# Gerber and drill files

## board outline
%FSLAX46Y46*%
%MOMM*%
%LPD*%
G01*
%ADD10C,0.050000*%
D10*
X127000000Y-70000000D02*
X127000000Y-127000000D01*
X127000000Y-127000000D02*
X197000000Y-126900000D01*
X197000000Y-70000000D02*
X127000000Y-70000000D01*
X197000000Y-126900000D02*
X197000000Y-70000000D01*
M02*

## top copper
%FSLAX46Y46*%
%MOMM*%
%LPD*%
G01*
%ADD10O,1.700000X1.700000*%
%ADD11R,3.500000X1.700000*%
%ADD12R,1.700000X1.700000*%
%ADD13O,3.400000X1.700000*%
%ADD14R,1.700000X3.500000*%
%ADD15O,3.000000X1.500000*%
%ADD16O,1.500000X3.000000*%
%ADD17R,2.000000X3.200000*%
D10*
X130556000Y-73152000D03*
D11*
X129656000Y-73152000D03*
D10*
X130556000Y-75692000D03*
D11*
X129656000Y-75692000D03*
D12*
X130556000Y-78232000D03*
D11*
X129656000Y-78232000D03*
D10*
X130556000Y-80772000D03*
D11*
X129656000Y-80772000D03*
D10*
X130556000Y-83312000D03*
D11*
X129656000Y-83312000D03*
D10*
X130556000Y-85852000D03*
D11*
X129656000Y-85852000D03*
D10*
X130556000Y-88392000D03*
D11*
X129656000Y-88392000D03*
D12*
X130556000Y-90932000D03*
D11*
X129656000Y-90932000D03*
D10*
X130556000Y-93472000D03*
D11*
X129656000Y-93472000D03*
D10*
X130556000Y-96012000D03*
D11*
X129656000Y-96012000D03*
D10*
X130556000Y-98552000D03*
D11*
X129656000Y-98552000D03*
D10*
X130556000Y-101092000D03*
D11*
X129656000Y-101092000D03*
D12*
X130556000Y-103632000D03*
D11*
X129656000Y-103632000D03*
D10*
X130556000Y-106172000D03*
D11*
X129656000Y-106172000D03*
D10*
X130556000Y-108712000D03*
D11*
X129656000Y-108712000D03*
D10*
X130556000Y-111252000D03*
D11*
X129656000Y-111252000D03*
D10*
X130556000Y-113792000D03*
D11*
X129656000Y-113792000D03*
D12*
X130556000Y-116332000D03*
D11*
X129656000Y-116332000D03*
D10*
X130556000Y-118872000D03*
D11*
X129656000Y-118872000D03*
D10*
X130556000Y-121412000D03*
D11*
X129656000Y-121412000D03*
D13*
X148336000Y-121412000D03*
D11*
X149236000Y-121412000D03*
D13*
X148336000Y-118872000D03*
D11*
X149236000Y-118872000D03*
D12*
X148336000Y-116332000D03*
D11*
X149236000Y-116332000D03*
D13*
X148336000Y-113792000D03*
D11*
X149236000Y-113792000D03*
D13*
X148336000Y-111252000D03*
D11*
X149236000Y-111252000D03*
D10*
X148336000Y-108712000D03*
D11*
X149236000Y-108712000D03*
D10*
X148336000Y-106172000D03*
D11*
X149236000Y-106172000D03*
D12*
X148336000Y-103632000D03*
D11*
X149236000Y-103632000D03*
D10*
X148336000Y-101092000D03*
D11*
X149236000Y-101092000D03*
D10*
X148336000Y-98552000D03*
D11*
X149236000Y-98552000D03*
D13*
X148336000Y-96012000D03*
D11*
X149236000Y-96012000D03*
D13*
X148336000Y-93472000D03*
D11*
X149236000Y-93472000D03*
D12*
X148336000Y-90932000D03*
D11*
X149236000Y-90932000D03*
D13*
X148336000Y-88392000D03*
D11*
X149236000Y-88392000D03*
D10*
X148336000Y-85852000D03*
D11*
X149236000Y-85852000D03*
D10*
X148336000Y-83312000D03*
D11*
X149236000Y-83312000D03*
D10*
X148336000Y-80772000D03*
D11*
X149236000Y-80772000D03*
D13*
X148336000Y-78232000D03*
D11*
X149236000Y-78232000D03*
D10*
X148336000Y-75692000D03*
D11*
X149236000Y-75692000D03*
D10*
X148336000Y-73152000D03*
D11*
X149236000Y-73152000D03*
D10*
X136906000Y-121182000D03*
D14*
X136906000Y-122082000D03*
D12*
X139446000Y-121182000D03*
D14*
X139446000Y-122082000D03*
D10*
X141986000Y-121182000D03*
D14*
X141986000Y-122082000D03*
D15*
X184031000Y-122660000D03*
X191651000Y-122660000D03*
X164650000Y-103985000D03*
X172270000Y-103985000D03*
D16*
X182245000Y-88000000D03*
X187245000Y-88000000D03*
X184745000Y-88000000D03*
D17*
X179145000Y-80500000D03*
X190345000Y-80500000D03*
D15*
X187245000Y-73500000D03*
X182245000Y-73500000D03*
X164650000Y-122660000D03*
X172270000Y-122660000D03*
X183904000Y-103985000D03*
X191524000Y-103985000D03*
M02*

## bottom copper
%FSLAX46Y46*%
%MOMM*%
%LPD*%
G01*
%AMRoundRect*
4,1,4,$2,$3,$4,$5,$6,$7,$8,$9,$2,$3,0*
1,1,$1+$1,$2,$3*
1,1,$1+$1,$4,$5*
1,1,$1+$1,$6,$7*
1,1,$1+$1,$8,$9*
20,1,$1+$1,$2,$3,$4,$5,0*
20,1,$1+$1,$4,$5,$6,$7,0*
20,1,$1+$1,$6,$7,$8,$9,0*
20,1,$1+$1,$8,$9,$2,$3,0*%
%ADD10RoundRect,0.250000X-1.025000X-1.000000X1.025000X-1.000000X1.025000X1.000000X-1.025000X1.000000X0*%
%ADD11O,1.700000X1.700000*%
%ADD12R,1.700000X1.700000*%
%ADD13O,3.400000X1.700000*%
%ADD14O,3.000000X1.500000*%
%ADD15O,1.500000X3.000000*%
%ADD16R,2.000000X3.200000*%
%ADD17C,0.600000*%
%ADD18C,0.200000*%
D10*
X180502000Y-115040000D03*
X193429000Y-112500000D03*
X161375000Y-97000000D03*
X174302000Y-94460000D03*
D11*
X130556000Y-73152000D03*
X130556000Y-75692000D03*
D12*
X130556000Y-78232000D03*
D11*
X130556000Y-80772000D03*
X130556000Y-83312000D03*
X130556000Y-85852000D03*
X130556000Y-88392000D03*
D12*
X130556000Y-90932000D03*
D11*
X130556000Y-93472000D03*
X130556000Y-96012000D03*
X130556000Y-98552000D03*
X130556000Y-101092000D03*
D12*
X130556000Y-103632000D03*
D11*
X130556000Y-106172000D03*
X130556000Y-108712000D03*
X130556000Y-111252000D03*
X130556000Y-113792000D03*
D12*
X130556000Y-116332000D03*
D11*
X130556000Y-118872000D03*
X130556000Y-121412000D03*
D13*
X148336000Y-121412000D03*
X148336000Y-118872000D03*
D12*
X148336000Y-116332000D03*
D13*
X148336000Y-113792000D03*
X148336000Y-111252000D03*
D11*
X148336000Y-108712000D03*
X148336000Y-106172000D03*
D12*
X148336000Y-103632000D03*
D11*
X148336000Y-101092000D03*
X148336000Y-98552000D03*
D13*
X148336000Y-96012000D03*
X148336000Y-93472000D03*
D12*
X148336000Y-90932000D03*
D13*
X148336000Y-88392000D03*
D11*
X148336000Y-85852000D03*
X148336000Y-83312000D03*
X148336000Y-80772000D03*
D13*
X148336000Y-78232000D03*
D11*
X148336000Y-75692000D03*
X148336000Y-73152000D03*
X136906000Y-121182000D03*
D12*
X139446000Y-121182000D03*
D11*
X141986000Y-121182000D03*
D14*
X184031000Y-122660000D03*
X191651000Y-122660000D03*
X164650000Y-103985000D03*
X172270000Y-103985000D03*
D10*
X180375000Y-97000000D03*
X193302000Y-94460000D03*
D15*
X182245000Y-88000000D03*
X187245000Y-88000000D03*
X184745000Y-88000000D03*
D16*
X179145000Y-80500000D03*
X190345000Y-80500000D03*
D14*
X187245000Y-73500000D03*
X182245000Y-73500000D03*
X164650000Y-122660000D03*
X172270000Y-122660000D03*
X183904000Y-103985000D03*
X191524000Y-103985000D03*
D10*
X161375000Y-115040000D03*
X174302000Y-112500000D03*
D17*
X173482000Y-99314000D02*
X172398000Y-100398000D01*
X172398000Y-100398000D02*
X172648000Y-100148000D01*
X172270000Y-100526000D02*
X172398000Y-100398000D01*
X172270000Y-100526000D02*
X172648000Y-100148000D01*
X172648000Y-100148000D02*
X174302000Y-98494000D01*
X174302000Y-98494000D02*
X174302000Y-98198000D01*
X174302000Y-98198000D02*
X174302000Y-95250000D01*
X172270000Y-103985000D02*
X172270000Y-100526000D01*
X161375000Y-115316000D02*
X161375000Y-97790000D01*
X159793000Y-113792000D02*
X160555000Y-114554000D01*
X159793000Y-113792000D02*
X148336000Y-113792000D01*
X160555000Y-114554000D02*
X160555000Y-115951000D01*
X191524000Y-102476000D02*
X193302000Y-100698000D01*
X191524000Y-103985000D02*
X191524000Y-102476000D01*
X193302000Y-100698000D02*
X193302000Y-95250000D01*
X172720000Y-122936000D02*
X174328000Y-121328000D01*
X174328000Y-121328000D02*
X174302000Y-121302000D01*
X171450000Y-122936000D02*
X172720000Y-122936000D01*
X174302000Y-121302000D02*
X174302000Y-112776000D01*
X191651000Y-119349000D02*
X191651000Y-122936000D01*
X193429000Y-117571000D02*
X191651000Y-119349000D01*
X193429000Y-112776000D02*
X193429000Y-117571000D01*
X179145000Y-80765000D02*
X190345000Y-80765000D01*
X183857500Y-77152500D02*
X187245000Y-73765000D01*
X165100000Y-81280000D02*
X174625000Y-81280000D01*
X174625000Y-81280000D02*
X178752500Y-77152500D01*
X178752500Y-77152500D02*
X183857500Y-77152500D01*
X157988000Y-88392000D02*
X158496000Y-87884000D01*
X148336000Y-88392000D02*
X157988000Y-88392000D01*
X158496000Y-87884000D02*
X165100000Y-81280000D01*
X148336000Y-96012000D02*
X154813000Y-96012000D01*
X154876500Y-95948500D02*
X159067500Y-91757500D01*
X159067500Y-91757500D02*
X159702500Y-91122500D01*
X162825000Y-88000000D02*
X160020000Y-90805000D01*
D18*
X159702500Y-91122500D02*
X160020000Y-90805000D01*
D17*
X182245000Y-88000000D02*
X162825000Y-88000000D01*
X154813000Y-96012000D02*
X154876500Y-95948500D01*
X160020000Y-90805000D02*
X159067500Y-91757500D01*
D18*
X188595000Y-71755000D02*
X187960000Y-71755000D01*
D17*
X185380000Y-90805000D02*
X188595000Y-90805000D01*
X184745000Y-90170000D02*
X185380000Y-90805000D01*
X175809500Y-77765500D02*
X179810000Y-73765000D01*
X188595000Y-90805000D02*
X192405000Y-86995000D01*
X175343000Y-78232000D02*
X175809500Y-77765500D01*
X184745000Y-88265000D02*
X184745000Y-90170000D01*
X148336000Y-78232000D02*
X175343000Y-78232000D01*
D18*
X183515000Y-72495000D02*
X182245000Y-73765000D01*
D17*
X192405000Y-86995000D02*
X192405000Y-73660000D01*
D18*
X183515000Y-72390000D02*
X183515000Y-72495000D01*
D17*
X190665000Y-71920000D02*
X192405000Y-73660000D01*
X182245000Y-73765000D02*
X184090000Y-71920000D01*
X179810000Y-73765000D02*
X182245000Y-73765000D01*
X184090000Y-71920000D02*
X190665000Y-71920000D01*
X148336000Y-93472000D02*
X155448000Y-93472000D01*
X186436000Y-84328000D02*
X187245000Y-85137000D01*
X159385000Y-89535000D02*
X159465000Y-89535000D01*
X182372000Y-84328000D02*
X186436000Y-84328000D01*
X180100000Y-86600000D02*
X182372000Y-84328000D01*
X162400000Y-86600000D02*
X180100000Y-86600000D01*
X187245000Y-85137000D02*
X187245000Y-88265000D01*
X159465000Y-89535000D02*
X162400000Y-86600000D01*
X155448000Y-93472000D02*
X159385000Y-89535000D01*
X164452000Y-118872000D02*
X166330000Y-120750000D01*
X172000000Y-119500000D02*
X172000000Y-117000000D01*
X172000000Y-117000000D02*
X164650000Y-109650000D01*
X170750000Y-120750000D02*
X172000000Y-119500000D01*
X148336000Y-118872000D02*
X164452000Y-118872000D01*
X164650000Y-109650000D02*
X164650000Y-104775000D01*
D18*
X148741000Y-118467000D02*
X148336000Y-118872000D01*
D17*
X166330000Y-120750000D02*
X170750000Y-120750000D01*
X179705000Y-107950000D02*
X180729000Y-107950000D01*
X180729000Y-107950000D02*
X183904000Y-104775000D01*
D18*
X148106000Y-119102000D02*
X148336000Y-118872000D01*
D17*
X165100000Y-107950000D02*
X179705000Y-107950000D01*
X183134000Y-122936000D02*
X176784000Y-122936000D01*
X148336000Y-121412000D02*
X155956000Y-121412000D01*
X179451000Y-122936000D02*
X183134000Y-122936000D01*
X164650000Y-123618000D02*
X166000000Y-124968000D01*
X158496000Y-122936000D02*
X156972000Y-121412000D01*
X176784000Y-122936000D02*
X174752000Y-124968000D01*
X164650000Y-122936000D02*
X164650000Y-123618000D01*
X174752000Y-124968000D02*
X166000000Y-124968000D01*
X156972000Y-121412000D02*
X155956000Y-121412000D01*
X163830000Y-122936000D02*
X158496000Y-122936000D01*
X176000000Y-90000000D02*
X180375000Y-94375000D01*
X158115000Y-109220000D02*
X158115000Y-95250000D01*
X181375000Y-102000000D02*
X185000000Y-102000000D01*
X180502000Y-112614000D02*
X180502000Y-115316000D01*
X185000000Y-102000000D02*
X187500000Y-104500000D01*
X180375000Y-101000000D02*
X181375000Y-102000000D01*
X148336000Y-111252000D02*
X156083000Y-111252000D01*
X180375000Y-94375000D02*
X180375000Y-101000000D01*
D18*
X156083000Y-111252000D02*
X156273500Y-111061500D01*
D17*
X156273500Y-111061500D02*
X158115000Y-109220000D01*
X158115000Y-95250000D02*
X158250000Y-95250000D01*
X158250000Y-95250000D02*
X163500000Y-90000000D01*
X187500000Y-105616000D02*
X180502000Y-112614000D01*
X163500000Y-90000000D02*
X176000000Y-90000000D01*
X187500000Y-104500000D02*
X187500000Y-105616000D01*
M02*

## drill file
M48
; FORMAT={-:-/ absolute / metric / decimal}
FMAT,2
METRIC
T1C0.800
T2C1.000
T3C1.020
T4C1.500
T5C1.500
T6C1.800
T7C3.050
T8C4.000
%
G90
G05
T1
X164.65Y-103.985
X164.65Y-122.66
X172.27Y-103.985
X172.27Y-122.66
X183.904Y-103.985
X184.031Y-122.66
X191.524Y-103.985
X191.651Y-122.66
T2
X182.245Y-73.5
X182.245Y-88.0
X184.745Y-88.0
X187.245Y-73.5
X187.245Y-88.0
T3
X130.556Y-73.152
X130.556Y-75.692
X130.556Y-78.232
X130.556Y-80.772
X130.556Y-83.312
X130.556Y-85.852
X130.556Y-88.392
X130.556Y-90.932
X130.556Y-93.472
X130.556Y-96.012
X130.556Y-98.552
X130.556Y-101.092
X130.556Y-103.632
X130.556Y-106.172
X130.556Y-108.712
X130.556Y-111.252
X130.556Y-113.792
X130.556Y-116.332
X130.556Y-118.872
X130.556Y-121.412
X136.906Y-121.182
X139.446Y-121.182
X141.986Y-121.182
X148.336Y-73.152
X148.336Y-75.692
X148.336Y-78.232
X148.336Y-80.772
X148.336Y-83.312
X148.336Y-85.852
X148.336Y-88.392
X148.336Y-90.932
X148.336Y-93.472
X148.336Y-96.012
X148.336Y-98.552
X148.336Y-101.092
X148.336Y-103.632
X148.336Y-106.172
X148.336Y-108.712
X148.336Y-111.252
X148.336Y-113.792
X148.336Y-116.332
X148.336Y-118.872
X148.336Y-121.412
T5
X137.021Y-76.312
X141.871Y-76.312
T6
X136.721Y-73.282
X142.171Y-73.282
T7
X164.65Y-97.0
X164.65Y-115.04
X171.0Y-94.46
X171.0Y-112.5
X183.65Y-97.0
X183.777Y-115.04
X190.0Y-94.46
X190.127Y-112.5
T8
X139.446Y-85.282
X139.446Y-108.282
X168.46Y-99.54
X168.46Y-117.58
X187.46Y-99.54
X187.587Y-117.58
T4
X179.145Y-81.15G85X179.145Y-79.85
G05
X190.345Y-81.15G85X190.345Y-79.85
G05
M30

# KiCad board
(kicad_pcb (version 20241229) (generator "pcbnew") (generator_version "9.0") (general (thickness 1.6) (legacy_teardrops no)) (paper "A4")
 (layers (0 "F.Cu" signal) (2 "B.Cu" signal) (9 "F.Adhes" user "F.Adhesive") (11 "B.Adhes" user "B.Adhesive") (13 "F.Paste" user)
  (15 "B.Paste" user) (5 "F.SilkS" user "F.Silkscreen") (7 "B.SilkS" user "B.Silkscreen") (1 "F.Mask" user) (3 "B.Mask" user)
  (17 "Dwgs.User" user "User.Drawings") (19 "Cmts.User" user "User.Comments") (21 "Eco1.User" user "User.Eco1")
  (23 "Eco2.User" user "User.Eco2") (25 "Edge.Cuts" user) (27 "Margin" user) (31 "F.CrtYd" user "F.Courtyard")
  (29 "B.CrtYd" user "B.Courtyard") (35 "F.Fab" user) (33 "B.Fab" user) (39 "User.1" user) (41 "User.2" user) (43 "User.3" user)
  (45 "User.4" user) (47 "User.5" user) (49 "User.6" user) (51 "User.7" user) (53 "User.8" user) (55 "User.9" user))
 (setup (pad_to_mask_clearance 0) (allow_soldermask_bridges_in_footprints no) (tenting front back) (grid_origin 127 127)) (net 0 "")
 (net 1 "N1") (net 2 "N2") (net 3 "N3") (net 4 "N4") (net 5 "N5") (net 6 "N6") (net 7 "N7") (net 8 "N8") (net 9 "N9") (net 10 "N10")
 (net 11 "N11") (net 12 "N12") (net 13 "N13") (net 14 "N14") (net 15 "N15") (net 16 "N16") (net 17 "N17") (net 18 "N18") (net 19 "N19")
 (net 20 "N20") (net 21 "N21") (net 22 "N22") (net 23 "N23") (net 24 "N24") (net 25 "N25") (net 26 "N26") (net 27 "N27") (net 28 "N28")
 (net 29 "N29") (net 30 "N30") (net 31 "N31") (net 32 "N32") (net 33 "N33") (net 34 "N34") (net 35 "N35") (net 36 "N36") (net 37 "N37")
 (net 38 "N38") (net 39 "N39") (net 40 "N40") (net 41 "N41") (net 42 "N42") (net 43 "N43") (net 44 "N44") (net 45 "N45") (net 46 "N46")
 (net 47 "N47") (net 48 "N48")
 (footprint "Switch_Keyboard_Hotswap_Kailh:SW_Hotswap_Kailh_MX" (layer "F.Cu") (at 187.587 117.58)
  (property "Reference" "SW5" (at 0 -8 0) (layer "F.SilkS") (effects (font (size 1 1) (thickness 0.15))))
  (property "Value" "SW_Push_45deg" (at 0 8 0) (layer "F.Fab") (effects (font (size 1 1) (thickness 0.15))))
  (pad "" np_thru_hole circle (at -3.81 -2.54) (size 3.05 3.05) (drill 3.05) (layers "*.Cu" "*.Mask"))
  (pad "" np_thru_hole circle (at 0 0) (size 4 4) (drill 4) (layers "*.Cu" "*.Mask"))
  (pad "" np_thru_hole circle (at 2.54 -5.08) (size 3.05 3.05) (drill 3.05) (layers "*.Cu" "*.Mask"))
  (pad "1" smd roundrect (at -7.085 -2.54) (size 2.55 2.5) (layers "B.Cu" "B.Mask" "B.Paste") (roundrect_rratio 0.1) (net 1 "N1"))
  (pad "2" smd roundrect (at 5.842 -5.08) (size 2.55 2.5) (layers "B.Cu" "B.Mask" "B.Paste") (roundrect_rratio 0.1) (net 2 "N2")))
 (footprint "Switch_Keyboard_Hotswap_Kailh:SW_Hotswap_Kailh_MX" (layer "F.Cu") (at 168.46 99.54)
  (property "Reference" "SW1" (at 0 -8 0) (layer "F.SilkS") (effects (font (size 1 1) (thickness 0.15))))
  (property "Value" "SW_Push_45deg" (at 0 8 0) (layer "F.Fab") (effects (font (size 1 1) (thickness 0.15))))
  (pad "" np_thru_hole circle (at -3.81 -2.54) (size 3.05 3.05) (drill 3.05) (layers "*.Cu" "*.Mask"))
  (pad "" np_thru_hole circle (at 0 0) (size 4 4) (drill 4) (layers "*.Cu" "*.Mask"))
  (pad "" np_thru_hole circle (at 2.54 -5.08) (size 3.05 3.05) (drill 3.05) (layers "*.Cu" "*.Mask"))
  (pad "1" smd roundrect (at -7.085 -2.54) (size 2.55 2.5) (layers "B.Cu" "B.Mask" "B.Paste") (roundrect_rratio 0.1) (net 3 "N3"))
  (pad "2" smd roundrect (at 5.842 -5.08) (size 2.55 2.5) (layers "B.Cu" "B.Mask" "B.Paste") (roundrect_rratio 0.1) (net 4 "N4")))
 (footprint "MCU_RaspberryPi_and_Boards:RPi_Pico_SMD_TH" (layer "F.Cu") (at 139.446 97.282)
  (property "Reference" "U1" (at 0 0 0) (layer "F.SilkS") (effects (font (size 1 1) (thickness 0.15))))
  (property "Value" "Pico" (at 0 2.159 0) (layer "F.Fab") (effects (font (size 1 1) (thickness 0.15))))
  (pad "" np_thru_hole oval (at -2.725 -24) (size 1.8 1.8) (drill 1.8) (layers "*.Cu" "*.Mask"))
  (pad "" np_thru_hole oval (at -2.425 -20.97) (size 1.5 1.5) (drill 1.5) (layers "*.Cu" "*.Mask"))
  (pad "" np_thru_hole oval (at 0 -12) (size 4 4) (drill 4) (layers "*.Cu" "*.Mask"))
  (pad "" np_thru_hole oval (at 0 11) (size 4 4) (drill 4) (layers "*.Cu" "*.Mask"))
  (pad "" np_thru_hole oval (at 2.425 -20.97) (size 1.5 1.5) (drill 1.5) (layers "*.Cu" "*.Mask"))
  (pad "" np_thru_hole oval (at 2.725 -24) (size 1.8 1.8) (drill 1.8) (layers "*.Cu" "*.Mask"))
  (pad "1" thru_hole oval (at -8.89 -24.13) (size 1.7 1.7) (drill 1.02) (layers "*.Cu" "*.Mask") (remove_unused_layers no) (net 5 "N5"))
  (pad "1" smd rect (at -8.89 -24.13) (size 3.5 1.7) (drill (offset -0.9 0)) (layers "F.Cu" "F.Mask") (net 5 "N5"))
  (pad "2" thru_hole oval (at -8.89 -21.59) (size 1.7 1.7) (drill 1.02) (layers "*.Cu" "*.Mask") (remove_unused_layers no) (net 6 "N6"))
  (pad "2" smd rect (at -8.89 -21.59) (size 3.5 1.7) (drill (offset -0.9 0)) (layers "F.Cu" "F.Mask") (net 6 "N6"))
  (pad "3" thru_hole rect (at -8.89 -19.05) (size 1.7 1.7) (drill 1.02) (layers "*.Cu" "*.Mask") (remove_unused_layers no) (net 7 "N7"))
  (pad "3" smd rect (at -8.89 -19.05) (size 3.5 1.7) (drill (offset -0.9 0)) (layers "F.Cu" "F.Mask") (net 7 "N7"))
  (pad "4" thru_hole oval (at -8.89 -16.51) (size 1.7 1.7) (drill 1.02) (layers "*.Cu" "*.Mask") (remove_unused_layers no) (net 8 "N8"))
  (pad "4" smd rect (at -8.89 -16.51) (size 3.5 1.7) (drill (offset -0.9 0)) (layers "F.Cu" "F.Mask") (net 8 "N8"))
  (pad "5" thru_hole oval (at -8.89 -13.97) (size 1.7 1.7) (drill 1.02) (layers "*.Cu" "*.Mask") (remove_unused_layers no) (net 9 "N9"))
  (pad "5" smd rect (at -8.89 -13.97) (size 3.5 1.7) (drill (offset -0.9 0)) (layers "F.Cu" "F.Mask") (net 9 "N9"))
  (pad "6" thru_hole oval (at -8.89 -11.43) (size 1.7 1.7) (drill 1.02) (layers "*.Cu" "*.Mask") (remove_unused_layers no) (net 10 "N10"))
  (pad "6" smd rect (at -8.89 -11.43) (size 3.5 1.7) (drill (offset -0.9 0)) (layers "F.Cu" "F.Mask") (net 10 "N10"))
  (pad "7" thru_hole oval (at -8.89 -8.89) (size 1.7 1.7) (drill 1.02) (layers "*.Cu" "*.Mask") (remove_unused_layers no) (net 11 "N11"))
  (pad "7" smd rect (at -8.89 -8.89) (size 3.5 1.7) (drill (offset -0.9 0)) (layers "F.Cu" "F.Mask") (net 11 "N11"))
  (pad "8" thru_hole rect (at -8.89 -6.35) (size 1.7 1.7) (drill 1.02) (layers "*.Cu" "*.Mask") (remove_unused_layers no) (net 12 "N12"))
  (pad "8" smd rect (at -8.89 -6.35) (size 3.5 1.7) (drill (offset -0.9 0)) (layers "F.Cu" "F.Mask") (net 12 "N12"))
  (pad "9" thru_hole oval (at -8.89 -3.81) (size 1.7 1.7) (drill 1.02) (layers "*.Cu" "*.Mask") (remove_unused_layers no) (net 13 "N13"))
  (pad "9" smd rect (at -8.89 -3.81) (size 3.5 1.7) (drill (offset -0.9 0)) (layers "F.Cu" "F.Mask") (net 13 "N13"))
  (pad "10" thru_hole oval (at -8.89 -1.27) (size 1.7 1.7) (drill 1.02) (layers "*.Cu" "*.Mask") (remove_unused_layers no) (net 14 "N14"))
  (pad "10" smd rect (at -8.89 -1.27) (size 3.5 1.7) (drill (offset -0.9 0)) (layers "F.Cu" "F.Mask") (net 14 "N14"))
  (pad "11" thru_hole oval (at -8.89 1.27) (size 1.7 1.7) (drill 1.02) (layers "*.Cu" "*.Mask") (remove_unused_layers no) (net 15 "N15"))
  (pad "11" smd rect (at -8.89 1.27) (size 3.5 1.7) (drill (offset -0.9 0)) (layers "F.Cu" "F.Mask") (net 15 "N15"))
  (pad "12" thru_hole oval (at -8.89 3.81) (size 1.7 1.7) (drill 1.02) (layers "*.Cu" "*.Mask") (remove_unused_layers no) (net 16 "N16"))
  (pad "12" smd rect (at -8.89 3.81) (size 3.5 1.7) (drill (offset -0.9 0)) (layers "F.Cu" "F.Mask") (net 16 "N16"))
  (pad "13" thru_hole rect (at -8.89 6.35) (size 1.7 1.7) (drill 1.02) (layers "*.Cu" "*.Mask") (remove_unused_layers no) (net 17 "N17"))
  (pad "13" smd rect (at -8.89 6.35) (size 3.5 1.7) (drill (offset -0.9 0)) (layers "F.Cu" "F.Mask") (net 17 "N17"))
  (pad "14" thru_hole oval (at -8.89 8.89) (size 1.7 1.7) (drill 1.02) (layers "*.Cu" "*.Mask") (remove_unused_layers no) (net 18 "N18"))
  (pad "14" smd rect (at -8.89 8.89) (size 3.5 1.7) (drill (offset -0.9 0)) (layers "F.Cu" "F.Mask") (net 18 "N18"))
  (pad "15" thru_hole oval (at -8.89 11.43) (size 1.7 1.7) (drill 1.02) (layers "*.Cu" "*.Mask") (remove_unused_layers no) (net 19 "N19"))
  (pad "15" smd rect (at -8.89 11.43) (size 3.5 1.7) (drill (offset -0.9 0)) (layers "F.Cu" "F.Mask") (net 19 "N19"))
  (pad "16" thru_hole oval (at -8.89 13.97) (size 1.7 1.7) (drill 1.02) (layers "*.Cu" "*.Mask") (remove_unused_layers no) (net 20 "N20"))
  (pad "16" smd rect (at -8.89 13.97) (size 3.5 1.7) (drill (offset -0.9 0)) (layers "F.Cu" "F.Mask") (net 20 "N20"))
  (pad "17" thru_hole oval (at -8.89 16.51) (size 1.7 1.7) (drill 1.02) (layers "*.Cu" "*.Mask") (remove_unused_layers no) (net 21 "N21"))
  (pad "17" smd rect (at -8.89 16.51) (size 3.5 1.7) (drill (offset -0.9 0)) (layers "F.Cu" "F.Mask") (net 21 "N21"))
  (pad "18" thru_hole rect (at -8.89 19.05) (size 1.7 1.7) (drill 1.02) (layers "*.Cu" "*.Mask") (remove_unused_layers no) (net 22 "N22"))
  (pad "18" smd rect (at -8.89 19.05) (size 3.5 1.7) (drill (offset -0.9 0)) (layers "F.Cu" "F.Mask") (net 22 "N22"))
  (pad "19" thru_hole oval (at -8.89 21.59) (size 1.7 1.7) (drill 1.02) (layers "*.Cu" "*.Mask") (remove_unused_layers no) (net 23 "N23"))
  (pad "19" smd rect (at -8.89 21.59) (size 3.5 1.7) (drill (offset -0.9 0)) (layers "F.Cu" "F.Mask") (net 23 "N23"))
  (pad "20" thru_hole oval (at -8.89 24.13) (size 1.7 1.7) (drill 1.02) (layers "*.Cu" "*.Mask") (remove_unused_layers no) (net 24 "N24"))
  (pad "20" smd rect (at -8.89 24.13) (size 3.5 1.7) (drill (offset -0.9 0)) (layers "F.Cu" "F.Mask") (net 24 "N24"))
  (pad "21" thru_hole oval (at 8.89 24.13) (size 3.4 1.7) (drill 1.02) (layers "*.Cu" "*.Mask") (remove_unused_layers no) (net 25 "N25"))
  (pad "21" smd rect (at 8.89 24.13) (size 3.5 1.7) (drill (offset 0.9 0)) (layers "F.Cu" "F.Mask") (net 25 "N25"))
  (pad "22" thru_hole oval (at 8.89 21.59) (size 3.4 1.7) (drill 1.02) (layers "*.Cu" "*.Mask") (remove_unused_layers no) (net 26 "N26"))
  (pad "22" smd rect (at 8.89 21.59) (size 3.5 1.7) (drill (offset 0.9 0)) (layers "F.Cu" "F.Mask") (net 26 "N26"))
  (pad "23" thru_hole rect (at 8.89 19.05) (size 1.7 1.7) (drill 1.02) (layers "*.Cu" "*.Mask") (remove_unused_layers no) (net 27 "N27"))
  (pad "23" smd rect (at 8.89 19.05) (size 3.5 1.7) (drill (offset 0.9 0)) (layers "F.Cu" "F.Mask") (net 27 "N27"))
  (pad "24" thru_hole oval (at 8.89 16.51) (size 3.4 1.7) (drill 1.02) (layers "*.Cu" "*.Mask") (remove_unused_layers no) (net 3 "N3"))
  (pad "24" smd rect (at 8.89 16.51) (size 3.5 1.7) (drill (offset 0.9 0)) (layers "F.Cu" "F.Mask") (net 3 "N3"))
  (pad "25" thru_hole oval (at 8.89 13.97) (size 3.4 1.7) (drill 1.02) (layers "*.Cu" "*.Mask") (remove_unused_layers no) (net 1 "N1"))
  (pad "25" smd rect (at 8.89 13.97) (size 3.5 1.7) (drill (offset 0.9 0)) (layers "F.Cu" "F.Mask") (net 1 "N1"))
  (pad "26" thru_hole oval (at 8.89 11.43) (size 1.7 1.7) (drill 1.02) (layers "*.Cu" "*.Mask") (remove_unused_layers no) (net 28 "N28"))
  (pad "26" smd rect (at 8.89 11.43) (size 3.5 1.7) (drill (offset 0.9 0)) (layers "F.Cu" "F.Mask") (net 28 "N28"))
  (pad "27" thru_hole oval (at 8.89 8.89) (size 1.7 1.7) (drill 1.02) (layers "*.Cu" "*.Mask") (remove_unused_layers no) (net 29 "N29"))
  (pad "27" smd rect (at 8.89 8.89) (size 3.5 1.7) (drill (offset 0.9 0)) (layers "F.Cu" "F.Mask") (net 29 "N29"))
  (pad "28" thru_hole rect (at 8.89 6.35) (size 1.7 1.7) (drill 1.02) (layers "*.Cu" "*.Mask") (remove_unused_layers no) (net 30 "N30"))
  (pad "28" smd rect (at 8.89 6.35) (size 3.5 1.7) (drill (offset 0.9 0)) (layers "F.Cu" "F.Mask") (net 30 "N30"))
  (pad "29" thru_hole oval (at 8.89 3.81) (size 1.7 1.7) (drill 1.02) (layers "*.Cu" "*.Mask") (remove_unused_layers no) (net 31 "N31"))
  (pad "29" smd rect (at 8.89 3.81) (size 3.5 1.7) (drill (offset 0.9 0)) (layers "F.Cu" "F.Mask") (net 31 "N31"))
  (pad "30" thru_hole oval (at 8.89 1.27) (size 1.7 1.7) (drill 1.02) (layers "*.Cu" "*.Mask") (remove_unused_layers no) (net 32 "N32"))
  (pad "30" smd rect (at 8.89 1.27) (size 3.5 1.7) (drill (offset 0.9 0)) (layers "F.Cu" "F.Mask") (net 32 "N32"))
  (pad "31" thru_hole oval (at 8.89 -1.27) (size 3.4 1.7) (drill 1.02) (layers "*.Cu" "*.Mask") (remove_unused_layers no) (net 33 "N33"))
  (pad "31" smd rect (at 8.89 -1.27) (size 3.5 1.7) (drill (offset 0.9 0)) (layers "F.Cu" "F.Mask") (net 33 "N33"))
  (pad "32" thru_hole oval (at 8.89 -3.81) (size 3.4 1.7) (drill 1.02) (layers "*.Cu" "*.Mask") (remove_unused_layers no) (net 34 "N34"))
  (pad "32" smd rect (at 8.89 -3.81) (size 3.5 1.7) (drill (offset 0.9 0)) (layers "F.Cu" "F.Mask") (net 34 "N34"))
  (pad "33" thru_hole rect (at 8.89 -6.35) (size 1.7 1.7) (drill 1.02) (layers "*.Cu" "*.Mask") (remove_unused_layers no) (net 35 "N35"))
  (pad "33" smd rect (at 8.89 -6.35) (size 3.5 1.7) (drill (offset 0.9 0)) (layers "F.Cu" "F.Mask") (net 35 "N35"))
  (pad "34" thru_hole oval (at 8.89 -8.89) (size 3.4 1.7) (drill 1.02) (layers "*.Cu" "*.Mask") (remove_unused_layers no) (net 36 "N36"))
  (pad "34" smd rect (at 8.89 -8.89) (size 3.5 1.7) (drill (offset 0.9 0)) (layers "F.Cu" "F.Mask") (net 36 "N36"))
  (pad "35" thru_hole oval (at 8.89 -11.43) (size 1.7 1.7) (drill 1.02) (layers "*.Cu" "*.Mask") (remove_unused_layers no) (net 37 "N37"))
  (pad "35" smd rect (at 8.89 -11.43) (size 3.5 1.7) (drill (offset 0.9 0)) (layers "F.Cu" "F.Mask") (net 37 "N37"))
  (pad "36" thru_hole oval (at 8.89 -13.97) (size 1.7 1.7) (drill 1.02) (layers "*.Cu" "*.Mask") (remove_unused_layers no) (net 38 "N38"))
  (pad "36" smd rect (at 8.89 -13.97) (size 3.5 1.7) (drill (offset 0.9 0)) (layers "F.Cu" "F.Mask") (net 38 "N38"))
  (pad "37" thru_hole oval (at 8.89 -16.51) (size 1.7 1.7) (drill 1.02) (layers "*.Cu" "*.Mask") (remove_unused_layers no) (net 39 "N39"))
  (pad "37" smd rect (at 8.89 -16.51) (size 3.5 1.7) (drill (offset 0.9 0)) (layers "F.Cu" "F.Mask") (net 39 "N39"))
  (pad "38" thru_hole oval (at 8.89 -19.05) (size 3.4 1.7) (drill 1.02) (layers "*.Cu" "*.Mask") (remove_unused_layers no) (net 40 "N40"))
  (pad "38" smd rect (at 8.89 -19.05) (size 3.5 1.7) (drill (offset 0.9 0)) (layers "F.Cu" "F.Mask") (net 40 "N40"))
  (pad "39" thru_hole oval (at 8.89 -21.59) (size 1.7 1.7) (drill 1.02) (layers "*.Cu" "*.Mask") (remove_unused_layers no) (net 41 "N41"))
  (pad "39" smd rect (at 8.89 -21.59) (size 3.5 1.7) (drill (offset 0.9 0)) (layers "F.Cu" "F.Mask") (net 41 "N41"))
  (pad "40" thru_hole oval (at 8.89 -24.13) (size 1.7 1.7) (drill 1.02) (layers "*.Cu" "*.Mask") (remove_unused_layers no) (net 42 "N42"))
  (pad "40" smd rect (at 8.89 -24.13) (size 3.5 1.7) (drill (offset 0.9 0)) (layers "F.Cu" "F.Mask") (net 42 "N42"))
  (pad "41" thru_hole oval (at -2.54 23.9) (size 1.7 1.7) (drill 1.02) (layers "*.Cu" "*.Mask") (remove_unused_layers no) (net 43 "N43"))
  (pad "41" smd rect (at -2.54 23.9 90) (size 3.5 1.7) (drill (offset -0.9 0)) (layers "F.Cu" "F.Mask") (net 43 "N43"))
  (pad "42" thru_hole rect (at 0 23.9) (size 1.7 1.7) (drill 1.02) (layers "*.Cu" "*.Mask") (remove_unused_layers no) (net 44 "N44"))
  (pad "42" smd rect (at 0 23.9 90) (size 3.5 1.7) (drill (offset -0.9 0)) (layers "F.Cu" "F.Mask") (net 44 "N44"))
  (pad "43" thru_hole oval (at 2.54 23.9) (size 1.7 1.7) (drill 1.02) (layers "*.Cu" "*.Mask") (remove_unused_layers no) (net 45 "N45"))
  (pad "43" smd rect (at 2.54 23.9 90) (size 3.5 1.7) (drill (offset -0.9 0)) (layers "F.Cu" "F.Mask") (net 45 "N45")))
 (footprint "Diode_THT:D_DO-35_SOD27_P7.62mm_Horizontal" (layer "F.Cu") (at 184.031 122.66)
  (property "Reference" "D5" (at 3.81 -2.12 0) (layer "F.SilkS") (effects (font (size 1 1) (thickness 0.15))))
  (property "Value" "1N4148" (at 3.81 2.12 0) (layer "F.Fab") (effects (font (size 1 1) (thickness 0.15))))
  (pad "1" thru_hole oval (at 0 0) (size 3 1.5) (drill 0.8) (layers "*.Cu" "*.Mask") (remove_unused_layers no) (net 25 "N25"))
  (pad "2" thru_hole oval (at 7.62 0) (size 3 1.5) (drill 0.8) (layers "*.Cu" "*.Mask") (remove_unused_layers no) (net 2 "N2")))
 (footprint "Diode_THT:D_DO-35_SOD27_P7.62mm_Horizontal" (layer "F.Cu") (at 164.65 103.985)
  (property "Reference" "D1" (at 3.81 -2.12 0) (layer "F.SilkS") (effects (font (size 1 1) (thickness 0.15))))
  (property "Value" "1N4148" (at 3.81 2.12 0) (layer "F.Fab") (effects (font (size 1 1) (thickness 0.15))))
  (pad "1" thru_hole oval (at 0 0) (size 3 1.5) (drill 0.8) (layers "*.Cu" "*.Mask") (remove_unused_layers no) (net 26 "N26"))
  (pad "2" thru_hole oval (at 7.62 0) (size 3 1.5) (drill 0.8) (layers "*.Cu" "*.Mask") (remove_unused_layers no) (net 4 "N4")))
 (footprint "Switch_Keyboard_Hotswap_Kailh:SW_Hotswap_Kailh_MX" (layer "F.Cu") (at 187.46 99.54)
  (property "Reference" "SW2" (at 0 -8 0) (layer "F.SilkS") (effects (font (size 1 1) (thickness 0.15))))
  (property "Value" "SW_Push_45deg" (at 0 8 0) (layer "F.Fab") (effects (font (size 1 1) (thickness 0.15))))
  (pad "" np_thru_hole circle (at -3.81 -2.54) (size 3.05 3.05) (drill 3.05) (layers "*.Cu" "*.Mask"))
  (pad "" np_thru_hole circle (at 0 0) (size 4 4) (drill 4) (layers "*.Cu" "*.Mask"))
  (pad "" np_thru_hole circle (at 2.54 -5.08) (size 3.05 3.05) (drill 3.05) (layers "*.Cu" "*.Mask"))
  (pad "1" smd roundrect (at -7.085 -2.54) (size 2.55 2.5) (layers "B.Cu" "B.Mask" "B.Paste") (roundrect_rratio 0.1) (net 1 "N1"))
  (pad "2" smd roundrect (at 5.842 -5.08) (size 2.55 2.5) (layers "B.Cu" "B.Mask" "B.Paste") (roundrect_rratio 0.1) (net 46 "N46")))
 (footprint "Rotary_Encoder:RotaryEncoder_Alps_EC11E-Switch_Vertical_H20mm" (layer "F.Cu") (at 182.245 88 90)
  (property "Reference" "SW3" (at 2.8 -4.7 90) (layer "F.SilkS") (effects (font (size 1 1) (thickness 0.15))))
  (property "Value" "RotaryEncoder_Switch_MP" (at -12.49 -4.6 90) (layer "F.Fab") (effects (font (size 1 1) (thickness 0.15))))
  (pad "A" thru_hole oval (at 0 0 90) (size 3 1.5) (drill 1) (layers "*.Cu" "*.Mask") (remove_unused_layers no) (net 33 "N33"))
  (pad "B" thru_hole oval (at 0 5 90) (size 3 1.5) (drill 1) (layers "*.Cu" "*.Mask") (remove_unused_layers no) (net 34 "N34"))
  (pad "C" thru_hole oval (at 0 2.5 90) (size 3 1.5) (drill 1) (layers "*.Cu" "*.Mask") (remove_unused_layers no) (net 40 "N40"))
  (pad "MP" thru_hole rect (at 7.5 -3.1 90) (size 3.2 2) (drill oval 2.8 1.5) (layers "*.Cu" "*.Mask") (remove_unused_layers no)
   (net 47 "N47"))
  (pad "MP" thru_hole rect (at 7.5 8.1 90) (size 3.2 2) (drill oval 2.8 1.5) (layers "*.Cu" "*.Mask") (remove_unused_layers no)
   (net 47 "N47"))
  (pad "S1" thru_hole oval (at 14.5 5 180) (size 3 1.5) (drill 1) (layers "*.Cu" "*.Mask") (remove_unused_layers no) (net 36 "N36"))
  (pad "S2" thru_hole oval (at 14.5 0 180) (size 3 1.5) (drill 1) (layers "*.Cu" "*.Mask") (remove_unused_layers no) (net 40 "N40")))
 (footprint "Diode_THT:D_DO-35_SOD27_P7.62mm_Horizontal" (layer "F.Cu") (at 164.65 122.66)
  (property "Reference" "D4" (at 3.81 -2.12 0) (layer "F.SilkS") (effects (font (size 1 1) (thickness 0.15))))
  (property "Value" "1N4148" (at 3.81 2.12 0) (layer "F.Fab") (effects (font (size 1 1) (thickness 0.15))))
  (pad "1" thru_hole oval (at 0 0) (size 3 1.5) (drill 0.8) (layers "*.Cu" "*.Mask") (remove_unused_layers no) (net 25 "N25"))
  (pad "2" thru_hole oval (at 7.62 0) (size 3 1.5) (drill 0.8) (layers "*.Cu" "*.Mask") (remove_unused_layers no) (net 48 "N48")))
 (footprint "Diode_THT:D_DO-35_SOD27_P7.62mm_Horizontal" (layer "F.Cu") (at 183.904 103.985)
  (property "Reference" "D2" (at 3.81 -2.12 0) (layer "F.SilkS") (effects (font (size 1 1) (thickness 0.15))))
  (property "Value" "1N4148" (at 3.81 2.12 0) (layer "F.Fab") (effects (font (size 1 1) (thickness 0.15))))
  (pad "1" thru_hole oval (at 0 0) (size 3 1.5) (drill 0.8) (layers "*.Cu" "*.Mask") (remove_unused_layers no) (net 26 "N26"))
  (pad "2" thru_hole oval (at 7.62 0) (size 3 1.5) (drill 0.8) (layers "*.Cu" "*.Mask") (remove_unused_layers no) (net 46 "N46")))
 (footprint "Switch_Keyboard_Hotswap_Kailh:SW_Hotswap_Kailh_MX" (layer "F.Cu") (at 168.46 117.58)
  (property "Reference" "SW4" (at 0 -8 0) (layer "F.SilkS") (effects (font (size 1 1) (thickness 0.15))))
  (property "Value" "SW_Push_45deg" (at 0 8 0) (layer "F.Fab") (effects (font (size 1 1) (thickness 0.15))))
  (pad "" np_thru_hole circle (at -3.81 -2.54) (size 3.05 3.05) (drill 3.05) (layers "*.Cu" "*.Mask"))
  (pad "" np_thru_hole circle (at 0 0) (size 4 4) (drill 4) (layers "*.Cu" "*.Mask"))
  (pad "" np_thru_hole circle (at 2.54 -5.08) (size 3.05 3.05) (drill 3.05) (layers "*.Cu" "*.Mask"))
  (pad "1" smd roundrect (at -7.085 -2.54) (size 2.55 2.5) (layers "B.Cu" "B.Mask" "B.Paste") (roundrect_rratio 0.1) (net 3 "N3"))
  (pad "2" smd roundrect (at 5.842 -5.08) (size 2.55 2.5) (layers "B.Cu" "B.Mask" "B.Paste") (roundrect_rratio 0.1) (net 48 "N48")))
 (gr_line (start 127 70) (end 127 127) (stroke (width 0.05) (type default)) (layer "Edge.Cuts"))
 (gr_line (start 127 127) (end 197 126.9) (stroke (width 0.05) (type default)) (layer "Edge.Cuts"))
 (gr_line (start 197 70) (end 127 70) (stroke (width 0.05) (type default)) (layer "Edge.Cuts"))
 (gr_line (start 197 126.9) (end 197 70) (stroke (width 0.05) (type default)) (layer "Edge.Cuts"))
 (segment (start 173.482 99.314) (end 172.398 100.398) (width 0.6) (layer "B.Cu") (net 4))
 (segment (start 172.398 100.398) (end 172.648 100.148) (width 0.6) (layer "B.Cu") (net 4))
 (segment (start 172.27 100.526) (end 172.398 100.398) (width 0.6) (layer "B.Cu") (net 4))
 (segment (start 172.27 100.526) (end 172.648 100.148) (width 0.6) (layer "B.Cu") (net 4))
 (segment (start 172.648 100.148) (end 174.302 98.494) (width 0.6) (layer "B.Cu") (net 4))
 (segment (start 174.302 98.494) (end 174.302 98.198) (width 0.6) (layer "B.Cu") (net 4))
 (segment (start 174.302 98.198) (end 174.302 95.25) (width 0.6) (layer "B.Cu") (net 4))
 (segment (start 172.27 103.985) (end 172.27 100.526) (width 0.6) (layer "B.Cu") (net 4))
 (segment (start 161.375 115.316) (end 161.375 97.79) (width 0.6) (layer "B.Cu") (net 3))
 (segment (start 159.793 113.792) (end 160.555 114.554) (width 0.6) (layer "B.Cu") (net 3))
 (segment (start 159.793 113.792) (end 148.336 113.792) (width 0.6) (layer "B.Cu") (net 3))
 (segment (start 160.555 114.554) (end 160.555 115.951) (width 0.6) (layer "B.Cu") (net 3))
 (segment (start 191.524 102.476) (end 193.302 100.698) (width 0.6) (layer "B.Cu") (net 46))
 (segment (start 191.524 103.985) (end 191.524 102.476) (width 0.6) (layer "B.Cu") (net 46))
 (segment (start 193.302 100.698) (end 193.302 95.25) (width 0.6) (layer "B.Cu") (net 46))
 (segment (start 172.72 122.936) (end 174.328 121.328) (width 0.6) (layer "B.Cu") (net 48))
 (segment (start 174.328 121.328) (end 174.302 121.302) (width 0.6) (layer "B.Cu") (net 48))
 (segment (start 171.45 122.936) (end 172.72 122.936) (width 0.6) (layer "B.Cu") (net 48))
 (segment (start 174.302 121.302) (end 174.302 112.776) (width 0.6) (layer "B.Cu") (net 48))
 (segment (start 191.651 119.349) (end 191.651 122.936) (width 0.6) (layer "B.Cu") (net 2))
 (segment (start 193.429 117.571) (end 191.651 119.349) (width 0.6) (layer "B.Cu") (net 2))
 (segment (start 193.429 112.776) (end 193.429 117.571) (width 0.6) (layer "B.Cu") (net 2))
 (segment (start 179.145 80.765) (end 190.345 80.765) (width 0.6) (layer "B.Cu") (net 47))
 (segment (start 183.8575 77.1525) (end 187.245 73.765) (width 0.6) (layer "B.Cu") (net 36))
 (segment (start 165.1 81.28) (end 174.625 81.28) (width 0.6) (layer "B.Cu") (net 36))
 (segment (start 174.625 81.28) (end 178.7525 77.1525) (width 0.6) (layer "B.Cu") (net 36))
 (segment (start 178.7525 77.1525) (end 183.8575 77.1525) (width 0.6) (layer "B.Cu") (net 36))
 (segment (start 157.988 88.392) (end 158.496 87.884) (width 0.6) (layer "B.Cu") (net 36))
 (segment (start 148.336 88.392) (end 157.988 88.392) (width 0.6) (layer "B.Cu") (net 36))
 (segment (start 158.496 87.884) (end 165.1 81.28) (width 0.6) (layer "B.Cu") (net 36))
 (segment (start 148.336 96.012) (end 154.813 96.012) (width 0.6) (layer "B.Cu") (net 33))
 (segment (start 154.8765 95.9485) (end 159.0675 91.7575) (width 0.6) (layer "B.Cu") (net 33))
 (segment (start 159.0675 91.7575) (end 159.7025 91.1225) (width 0.6) (layer "B.Cu") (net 33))
 (segment (start 162.825 88) (end 160.02 90.805) (width 0.6) (layer "B.Cu") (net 33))
 (segment (start 159.7025 91.1225) (end 160.02 90.805) (width 0.2) (layer "B.Cu") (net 33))
 (segment (start 182.245 88) (end 162.825 88) (width 0.6) (layer "B.Cu") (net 33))
 (segment (start 154.813 96.012) (end 154.8765 95.9485) (width 0.6) (layer "B.Cu") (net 33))
 (segment (start 160.02 90.805) (end 159.0675 91.7575) (width 0.6) (layer "B.Cu") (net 33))
 (segment (start 188.595 71.755) (end 187.96 71.755) (width 0.2) (layer "B.Cu") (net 40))
 (segment (start 185.38 90.805) (end 188.595 90.805) (width 0.6) (layer "B.Cu") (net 40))
 (segment (start 184.745 90.17) (end 185.38 90.805) (width 0.6) (layer "B.Cu") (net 40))
 (segment (start 175.8095 77.7655) (end 179.81 73.765) (width 0.6) (layer "B.Cu") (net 40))
 (segment (start 188.595 90.805) (end 192.405 86.995) (width 0.6) (layer "B.Cu") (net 40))
 (segment (start 175.343 78.232) (end 175.8095 77.7655) (width 0.6) (layer "B.Cu") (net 40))
 (segment (start 184.745 88.265) (end 184.745 90.17) (width 0.6) (layer "B.Cu") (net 40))
 (segment (start 148.336 78.232) (end 175.343 78.232) (width 0.6) (layer "B.Cu") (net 40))
 (segment (start 183.515 72.495) (end 182.245 73.765) (width 0.2) (layer "B.Cu") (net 40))
 (segment (start 192.405 86.995) (end 192.405 73.66) (width 0.6) (layer "B.Cu") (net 40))
 (segment (start 183.515 72.39) (end 183.515 72.495) (width 0.2) (layer "B.Cu") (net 40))
 (segment (start 190.665 71.92) (end 192.405 73.66) (width 0.6) (layer "B.Cu") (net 40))
 (segment (start 182.245 73.765) (end 184.09 71.92) (width 0.6) (layer "B.Cu") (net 40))
 (segment (start 179.81 73.765) (end 182.245 73.765) (width 0.6) (layer "B.Cu") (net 40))
 (segment (start 184.09 71.92) (end 190.665 71.92) (width 0.6) (layer "B.Cu") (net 40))
 (segment (start 148.336 93.472) (end 155.448 93.472) (width 0.6) (layer "B.Cu") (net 34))
 (segment (start 186.436 84.328) (end 187.245 85.137) (width 0.6) (layer "B.Cu") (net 34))
 (segment (start 159.385 89.535) (end 159.465 89.535) (width 0.6) (layer "B.Cu") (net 34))
 (segment (start 182.372 84.328) (end 186.436 84.328) (width 0.6) (layer "B.Cu") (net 34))
 (segment (start 180.1 86.6) (end 182.372 84.328) (width 0.6) (layer "B.Cu") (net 34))
 (segment (start 162.4 86.6) (end 180.1 86.6) (width 0.6) (layer "B.Cu") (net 34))
 (segment (start 187.245 85.137) (end 187.245 88.265) (width 0.6) (layer "B.Cu") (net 34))
 (segment (start 159.465 89.535) (end 162.4 86.6) (width 0.6) (layer "B.Cu") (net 34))
 (segment (start 155.448 93.472) (end 159.385 89.535) (width 0.6) (layer "B.Cu") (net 34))
 (segment (start 164.452 118.872) (end 166.33 120.75) (width 0.6) (layer "B.Cu") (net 26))
 (segment (start 172 119.5) (end 172 117) (width 0.6) (layer "B.Cu") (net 26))
 (segment (start 172 117) (end 164.65 109.65) (width 0.6) (layer "B.Cu") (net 26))
 (segment (start 170.75 120.75) (end 172 119.5) (width 0.6) (layer "B.Cu") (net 26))
 (segment (start 148.336 118.872) (end 164.452 118.872) (width 0.6) (layer "B.Cu") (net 26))
 (segment (start 164.65 109.65) (end 164.65 104.775) (width 0.6) (layer "B.Cu") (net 26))
 (segment (start 148.741 118.467) (end 148.336 118.872) (width 0.2) (layer "B.Cu") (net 26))
 (segment (start 166.33 120.75) (end 170.75 120.75) (width 0.6) (layer "B.Cu") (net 26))
 (segment (start 179.705 107.95) (end 180.729 107.95) (width 0.6) (layer "B.Cu") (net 26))
 (segment (start 180.729 107.95) (end 183.904 104.775) (width 0.6) (layer "B.Cu") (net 26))
 (segment (start 148.106 119.102) (end 148.336 118.872) (width 0.2) (layer "B.Cu") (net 26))
 (segment (start 165.1 107.95) (end 179.705 107.95) (width 0.6) (layer "B.Cu") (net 26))
 (segment (start 183.134 122.936) (end 176.784 122.936) (width 0.6) (layer "B.Cu") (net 25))
 (segment (start 148.336 121.412) (end 155.956 121.412) (width 0.6) (layer "B.Cu") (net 25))
 (segment (start 179.451 122.936) (end 183.134 122.936) (width 0.6) (layer "B.Cu") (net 25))
 (segment (start 164.65 123.618) (end 166 124.968) (width 0.6) (layer "B.Cu") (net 25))
 (segment (start 158.496 122.936) (end 156.972 121.412) (width 0.6) (layer "B.Cu") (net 25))
 (segment (start 176.784 122.936) (end 174.752 124.968) (width 0.6) (layer "B.Cu") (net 25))
 (segment (start 164.65 122.936) (end 164.65 123.618) (width 0.6) (layer "B.Cu") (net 25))
 (segment (start 174.752 124.968) (end 166 124.968) (width 0.6) (layer "B.Cu") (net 25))
 (segment (start 156.972 121.412) (end 155.956 121.412) (width 0.6) (layer "B.Cu") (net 25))
 (segment (start 163.83 122.936) (end 158.496 122.936) (width 0.6) (layer "B.Cu") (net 25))
 (segment (start 176 90) (end 180.375 94.375) (width 0.6) (layer "B.Cu") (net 1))
 (segment (start 158.115 109.22) (end 158.115 95.25) (width 0.6) (layer "B.Cu") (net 1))
 (segment (start 181.375 102) (end 185 102) (width 0.6) (layer "B.Cu") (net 1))
 (segment (start 180.502 112.614) (end 180.502 115.316) (width 0.6) (layer "B.Cu") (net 1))
 (segment (start 185 102) (end 187.5 104.5) (width 0.6) (layer "B.Cu") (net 1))
 (segment (start 180.375 101) (end 181.375 102) (width 0.6) (layer "B.Cu") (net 1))
 (segment (start 148.336 111.252) (end 156.083 111.252) (width 0.6) (layer "B.Cu") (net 1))
 (segment (start 180.375 94.375) (end 180.375 101) (width 0.6) (layer "B.Cu") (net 1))
 (segment (start 156.083 111.252) (end 156.2735 111.0615) (width 0.2) (layer "B.Cu") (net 1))
 (segment (start 156.2735 111.0615) (end 158.115 109.22) (width 0.6) (layer "B.Cu") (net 1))
 (segment (start 158.115 95.25) (end 158.25 95.25) (width 0.6) (layer "B.Cu") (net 1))
 (segment (start 158.25 95.25) (end 163.5 90) (width 0.6) (layer "B.Cu") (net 1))
 (segment (start 187.5 105.616) (end 180.502 112.614) (width 0.6) (layer "B.Cu") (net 1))
 (segment (start 163.5 90) (end 176 90) (width 0.6) (layer "B.Cu") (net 1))
 (segment (start 187.5 104.5) (end 187.5 105.616) (width 0.6) (layer "B.Cu") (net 1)))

